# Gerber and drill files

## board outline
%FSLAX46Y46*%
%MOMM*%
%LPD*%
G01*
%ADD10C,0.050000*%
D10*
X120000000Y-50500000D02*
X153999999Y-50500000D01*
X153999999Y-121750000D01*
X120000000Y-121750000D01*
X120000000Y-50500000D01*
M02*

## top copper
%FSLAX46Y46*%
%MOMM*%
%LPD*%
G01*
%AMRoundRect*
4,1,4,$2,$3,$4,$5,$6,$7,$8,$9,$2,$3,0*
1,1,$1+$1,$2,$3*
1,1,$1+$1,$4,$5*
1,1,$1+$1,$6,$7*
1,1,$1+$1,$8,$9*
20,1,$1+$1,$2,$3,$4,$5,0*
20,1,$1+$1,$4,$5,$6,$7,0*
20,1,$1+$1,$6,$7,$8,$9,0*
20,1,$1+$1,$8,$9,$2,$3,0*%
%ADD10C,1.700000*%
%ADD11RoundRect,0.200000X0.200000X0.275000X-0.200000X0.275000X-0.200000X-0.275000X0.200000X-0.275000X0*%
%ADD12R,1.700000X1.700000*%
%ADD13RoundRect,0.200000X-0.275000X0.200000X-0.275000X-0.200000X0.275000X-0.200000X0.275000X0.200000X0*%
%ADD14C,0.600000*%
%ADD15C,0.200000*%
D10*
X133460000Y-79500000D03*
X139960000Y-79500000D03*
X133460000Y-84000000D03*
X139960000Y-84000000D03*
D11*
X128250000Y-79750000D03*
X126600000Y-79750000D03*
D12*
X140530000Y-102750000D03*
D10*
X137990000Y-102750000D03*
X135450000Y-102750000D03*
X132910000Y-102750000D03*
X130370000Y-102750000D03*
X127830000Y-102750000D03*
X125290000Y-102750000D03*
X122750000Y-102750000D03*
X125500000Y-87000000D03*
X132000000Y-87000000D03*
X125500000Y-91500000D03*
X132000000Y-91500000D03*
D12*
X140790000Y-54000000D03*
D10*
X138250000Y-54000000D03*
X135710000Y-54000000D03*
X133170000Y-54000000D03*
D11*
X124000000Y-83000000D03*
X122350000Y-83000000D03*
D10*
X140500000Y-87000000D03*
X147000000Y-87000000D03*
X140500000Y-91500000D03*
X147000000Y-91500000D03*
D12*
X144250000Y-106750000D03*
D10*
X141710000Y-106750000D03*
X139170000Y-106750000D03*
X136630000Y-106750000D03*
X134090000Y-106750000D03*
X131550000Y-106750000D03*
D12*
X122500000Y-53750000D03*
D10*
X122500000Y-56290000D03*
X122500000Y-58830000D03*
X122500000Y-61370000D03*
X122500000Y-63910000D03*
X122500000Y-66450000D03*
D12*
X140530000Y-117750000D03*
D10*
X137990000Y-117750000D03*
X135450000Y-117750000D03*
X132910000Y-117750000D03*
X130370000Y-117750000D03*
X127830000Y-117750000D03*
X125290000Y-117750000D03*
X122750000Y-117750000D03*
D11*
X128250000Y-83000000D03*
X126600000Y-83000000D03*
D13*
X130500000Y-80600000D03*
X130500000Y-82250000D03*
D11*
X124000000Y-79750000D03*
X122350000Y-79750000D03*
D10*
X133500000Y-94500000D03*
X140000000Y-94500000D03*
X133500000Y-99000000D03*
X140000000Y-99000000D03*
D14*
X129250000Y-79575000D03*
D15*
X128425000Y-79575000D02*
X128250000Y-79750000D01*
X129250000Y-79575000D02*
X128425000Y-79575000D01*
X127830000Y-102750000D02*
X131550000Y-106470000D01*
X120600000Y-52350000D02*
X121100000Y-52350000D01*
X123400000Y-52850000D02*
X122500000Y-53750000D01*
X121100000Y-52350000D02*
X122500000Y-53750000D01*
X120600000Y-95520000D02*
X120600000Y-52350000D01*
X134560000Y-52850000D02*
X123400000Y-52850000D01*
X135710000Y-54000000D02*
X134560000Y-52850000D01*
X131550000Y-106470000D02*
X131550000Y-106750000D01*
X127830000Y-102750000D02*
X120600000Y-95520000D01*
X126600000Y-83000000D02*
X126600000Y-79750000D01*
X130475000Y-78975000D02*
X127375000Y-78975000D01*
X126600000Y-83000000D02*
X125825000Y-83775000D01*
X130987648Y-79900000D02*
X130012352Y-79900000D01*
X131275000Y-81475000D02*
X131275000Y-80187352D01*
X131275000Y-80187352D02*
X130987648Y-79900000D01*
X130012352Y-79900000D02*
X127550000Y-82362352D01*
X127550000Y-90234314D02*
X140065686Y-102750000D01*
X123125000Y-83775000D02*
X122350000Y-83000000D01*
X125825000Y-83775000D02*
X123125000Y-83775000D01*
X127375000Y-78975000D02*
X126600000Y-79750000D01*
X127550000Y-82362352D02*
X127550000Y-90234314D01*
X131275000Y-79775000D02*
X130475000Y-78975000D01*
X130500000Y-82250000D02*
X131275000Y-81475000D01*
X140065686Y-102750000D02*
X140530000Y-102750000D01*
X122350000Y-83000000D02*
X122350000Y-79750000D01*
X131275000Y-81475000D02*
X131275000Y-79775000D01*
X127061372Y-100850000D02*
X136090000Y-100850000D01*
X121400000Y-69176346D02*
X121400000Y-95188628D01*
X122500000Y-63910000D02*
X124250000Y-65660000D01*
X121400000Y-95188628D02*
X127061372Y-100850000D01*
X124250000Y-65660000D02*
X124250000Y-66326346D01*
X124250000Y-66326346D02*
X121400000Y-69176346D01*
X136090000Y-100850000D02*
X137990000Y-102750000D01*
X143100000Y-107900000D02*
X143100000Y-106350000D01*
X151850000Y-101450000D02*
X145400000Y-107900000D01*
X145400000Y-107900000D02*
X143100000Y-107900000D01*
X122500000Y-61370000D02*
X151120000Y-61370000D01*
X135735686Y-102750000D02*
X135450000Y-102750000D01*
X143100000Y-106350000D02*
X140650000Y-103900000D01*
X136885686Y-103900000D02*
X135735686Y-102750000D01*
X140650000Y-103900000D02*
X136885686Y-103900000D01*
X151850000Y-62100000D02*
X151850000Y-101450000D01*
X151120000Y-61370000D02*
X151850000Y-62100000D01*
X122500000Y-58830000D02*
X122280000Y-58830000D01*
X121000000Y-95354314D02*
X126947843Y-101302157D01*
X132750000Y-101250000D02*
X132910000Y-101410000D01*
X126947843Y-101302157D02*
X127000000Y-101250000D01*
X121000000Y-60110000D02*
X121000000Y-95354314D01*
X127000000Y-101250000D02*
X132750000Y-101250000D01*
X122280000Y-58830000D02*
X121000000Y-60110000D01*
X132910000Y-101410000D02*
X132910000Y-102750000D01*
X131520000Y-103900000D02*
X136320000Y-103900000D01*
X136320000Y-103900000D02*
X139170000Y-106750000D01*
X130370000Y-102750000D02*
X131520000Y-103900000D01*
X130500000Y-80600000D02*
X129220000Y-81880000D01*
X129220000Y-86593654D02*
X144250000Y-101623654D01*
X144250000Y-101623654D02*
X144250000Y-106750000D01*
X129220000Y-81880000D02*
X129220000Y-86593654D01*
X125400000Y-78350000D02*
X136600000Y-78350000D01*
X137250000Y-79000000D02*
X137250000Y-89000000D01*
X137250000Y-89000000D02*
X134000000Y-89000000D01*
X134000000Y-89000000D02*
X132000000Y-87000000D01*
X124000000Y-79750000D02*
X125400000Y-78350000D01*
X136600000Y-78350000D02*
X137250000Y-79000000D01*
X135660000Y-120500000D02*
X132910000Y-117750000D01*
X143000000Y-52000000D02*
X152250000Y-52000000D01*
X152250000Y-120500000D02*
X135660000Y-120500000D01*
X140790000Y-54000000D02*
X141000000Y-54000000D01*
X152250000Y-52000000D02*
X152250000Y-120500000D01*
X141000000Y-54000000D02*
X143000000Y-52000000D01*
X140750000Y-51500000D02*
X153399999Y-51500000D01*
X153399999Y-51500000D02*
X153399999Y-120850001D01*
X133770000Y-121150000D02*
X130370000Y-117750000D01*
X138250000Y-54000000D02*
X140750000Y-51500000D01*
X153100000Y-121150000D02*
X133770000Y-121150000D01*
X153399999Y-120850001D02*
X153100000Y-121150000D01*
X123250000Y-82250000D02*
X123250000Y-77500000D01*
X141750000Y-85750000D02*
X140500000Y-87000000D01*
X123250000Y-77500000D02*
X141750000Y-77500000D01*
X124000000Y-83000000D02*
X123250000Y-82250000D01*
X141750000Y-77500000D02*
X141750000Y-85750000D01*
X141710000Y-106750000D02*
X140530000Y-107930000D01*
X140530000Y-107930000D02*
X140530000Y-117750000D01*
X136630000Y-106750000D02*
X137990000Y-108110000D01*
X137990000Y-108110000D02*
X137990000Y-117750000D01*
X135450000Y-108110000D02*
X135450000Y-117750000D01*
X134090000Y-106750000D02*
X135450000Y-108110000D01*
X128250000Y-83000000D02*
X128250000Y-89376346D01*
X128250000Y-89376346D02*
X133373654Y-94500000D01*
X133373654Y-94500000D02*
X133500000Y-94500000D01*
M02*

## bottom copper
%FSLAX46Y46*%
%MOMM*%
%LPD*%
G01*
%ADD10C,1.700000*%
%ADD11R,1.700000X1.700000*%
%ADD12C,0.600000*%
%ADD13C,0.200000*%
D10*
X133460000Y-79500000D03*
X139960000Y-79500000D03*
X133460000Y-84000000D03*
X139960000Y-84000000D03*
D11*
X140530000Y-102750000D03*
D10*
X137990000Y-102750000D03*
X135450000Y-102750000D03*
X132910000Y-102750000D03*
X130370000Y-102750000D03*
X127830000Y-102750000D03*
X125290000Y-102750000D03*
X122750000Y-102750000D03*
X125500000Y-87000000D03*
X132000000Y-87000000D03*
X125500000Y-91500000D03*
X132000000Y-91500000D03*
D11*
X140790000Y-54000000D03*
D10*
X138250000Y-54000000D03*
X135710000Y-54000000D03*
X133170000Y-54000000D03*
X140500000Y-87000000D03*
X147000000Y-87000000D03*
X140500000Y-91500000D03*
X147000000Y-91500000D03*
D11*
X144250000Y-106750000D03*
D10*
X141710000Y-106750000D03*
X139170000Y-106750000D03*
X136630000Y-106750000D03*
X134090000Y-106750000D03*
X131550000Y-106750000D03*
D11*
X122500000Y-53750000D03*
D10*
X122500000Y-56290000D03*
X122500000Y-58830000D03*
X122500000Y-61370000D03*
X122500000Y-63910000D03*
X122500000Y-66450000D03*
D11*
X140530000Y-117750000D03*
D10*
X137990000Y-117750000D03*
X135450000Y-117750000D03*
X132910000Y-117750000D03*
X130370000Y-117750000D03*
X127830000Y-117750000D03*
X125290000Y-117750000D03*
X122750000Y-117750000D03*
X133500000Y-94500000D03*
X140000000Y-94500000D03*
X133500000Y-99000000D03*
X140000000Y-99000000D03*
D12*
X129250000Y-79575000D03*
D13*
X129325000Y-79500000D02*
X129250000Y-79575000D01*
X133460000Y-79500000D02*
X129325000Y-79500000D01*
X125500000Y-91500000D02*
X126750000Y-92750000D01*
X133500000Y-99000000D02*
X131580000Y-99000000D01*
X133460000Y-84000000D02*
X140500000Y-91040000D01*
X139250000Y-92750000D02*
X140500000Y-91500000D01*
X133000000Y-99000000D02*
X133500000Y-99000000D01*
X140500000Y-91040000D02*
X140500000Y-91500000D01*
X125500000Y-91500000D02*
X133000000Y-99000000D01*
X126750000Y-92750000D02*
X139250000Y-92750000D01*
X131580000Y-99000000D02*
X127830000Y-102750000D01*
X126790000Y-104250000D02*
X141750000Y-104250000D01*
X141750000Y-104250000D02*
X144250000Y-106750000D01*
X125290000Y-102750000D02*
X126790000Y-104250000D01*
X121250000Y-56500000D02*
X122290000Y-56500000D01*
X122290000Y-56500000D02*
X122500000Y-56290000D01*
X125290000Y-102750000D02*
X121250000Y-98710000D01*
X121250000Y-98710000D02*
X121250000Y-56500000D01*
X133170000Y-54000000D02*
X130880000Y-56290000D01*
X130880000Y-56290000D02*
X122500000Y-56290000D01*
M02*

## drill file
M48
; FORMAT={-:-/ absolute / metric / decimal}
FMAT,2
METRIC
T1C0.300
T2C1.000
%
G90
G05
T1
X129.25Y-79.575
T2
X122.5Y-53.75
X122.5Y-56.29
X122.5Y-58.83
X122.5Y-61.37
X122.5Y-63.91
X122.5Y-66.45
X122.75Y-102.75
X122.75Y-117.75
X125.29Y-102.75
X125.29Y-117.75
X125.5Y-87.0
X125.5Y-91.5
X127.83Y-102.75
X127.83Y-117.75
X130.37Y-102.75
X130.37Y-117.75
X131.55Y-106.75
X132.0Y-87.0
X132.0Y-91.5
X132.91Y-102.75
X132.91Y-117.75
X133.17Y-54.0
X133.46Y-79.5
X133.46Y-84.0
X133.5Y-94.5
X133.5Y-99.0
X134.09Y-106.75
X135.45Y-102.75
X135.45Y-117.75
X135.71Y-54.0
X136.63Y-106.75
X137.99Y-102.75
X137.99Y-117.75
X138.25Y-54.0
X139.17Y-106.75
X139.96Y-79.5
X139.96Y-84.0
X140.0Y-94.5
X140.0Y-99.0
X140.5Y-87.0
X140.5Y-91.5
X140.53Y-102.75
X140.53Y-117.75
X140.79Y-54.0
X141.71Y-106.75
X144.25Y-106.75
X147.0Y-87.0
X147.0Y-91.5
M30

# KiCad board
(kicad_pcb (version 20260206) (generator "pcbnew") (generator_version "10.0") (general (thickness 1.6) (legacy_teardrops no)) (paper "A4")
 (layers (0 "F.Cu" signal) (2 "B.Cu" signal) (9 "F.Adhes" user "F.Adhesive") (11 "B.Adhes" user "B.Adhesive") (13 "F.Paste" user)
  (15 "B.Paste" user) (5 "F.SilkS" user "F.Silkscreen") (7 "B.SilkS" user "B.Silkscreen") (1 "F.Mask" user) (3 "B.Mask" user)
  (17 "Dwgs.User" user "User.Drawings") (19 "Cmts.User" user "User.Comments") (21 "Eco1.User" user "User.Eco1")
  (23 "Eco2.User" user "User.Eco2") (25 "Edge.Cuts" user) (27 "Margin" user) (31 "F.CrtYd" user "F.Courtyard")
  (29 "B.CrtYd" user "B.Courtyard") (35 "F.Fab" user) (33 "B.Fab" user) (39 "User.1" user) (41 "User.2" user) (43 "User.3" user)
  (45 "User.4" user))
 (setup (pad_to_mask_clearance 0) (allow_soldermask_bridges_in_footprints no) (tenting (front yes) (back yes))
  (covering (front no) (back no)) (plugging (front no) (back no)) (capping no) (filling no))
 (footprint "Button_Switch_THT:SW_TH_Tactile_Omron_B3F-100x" (layer "F.Cu") (at 133.46 79.5)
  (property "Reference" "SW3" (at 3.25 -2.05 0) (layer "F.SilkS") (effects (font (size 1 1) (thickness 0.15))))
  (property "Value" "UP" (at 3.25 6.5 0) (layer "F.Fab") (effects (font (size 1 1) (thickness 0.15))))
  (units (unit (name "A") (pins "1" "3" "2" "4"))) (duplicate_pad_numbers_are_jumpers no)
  (pad "1" thru_hole circle (at 0 0) (size 1.7 1.7) (drill 1) (layers "*.Cu" "*.Mask") (remove_unused_layers no) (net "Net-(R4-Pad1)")
   (thermal_bridge_angle 90))
  (pad "1" thru_hole circle (at 6.5 0) (size 1.7 1.7) (drill 1) (layers "*.Cu" "*.Mask") (remove_unused_layers no) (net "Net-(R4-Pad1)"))
  (pad "2" thru_hole circle (at 0 4.5) (size 1.7 1.7) (drill 1) (layers "*.Cu" "*.Mask") (remove_unused_layers no) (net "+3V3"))
  (pad "2" thru_hole circle (at 6.5 4.5) (size 1.7 1.7) (drill 1) (layers "*.Cu" "*.Mask") (remove_unused_layers no)
   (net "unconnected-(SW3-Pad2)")))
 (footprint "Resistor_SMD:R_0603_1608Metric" (layer "F.Cu") (at 127.425 79.75 180)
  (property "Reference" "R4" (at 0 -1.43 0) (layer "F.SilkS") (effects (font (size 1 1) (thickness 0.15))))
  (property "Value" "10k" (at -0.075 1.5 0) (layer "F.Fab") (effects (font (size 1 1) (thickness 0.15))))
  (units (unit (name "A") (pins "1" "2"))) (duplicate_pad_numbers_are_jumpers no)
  (pad "1" smd roundrect (at -0.825 0 180) (size 0.8 0.95) (layers "F.Cu" "F.Mask" "F.Paste") (roundrect_rratio 0.25) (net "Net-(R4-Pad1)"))
  (pad "2" smd roundrect (at 0.825 0 180) (size 0.8 0.95) (layers "F.Cu" "F.Mask" "F.Paste") (roundrect_rratio 0.25) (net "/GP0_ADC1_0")))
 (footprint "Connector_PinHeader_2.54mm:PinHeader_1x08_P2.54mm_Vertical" (layer "F.Cu") (at 140.53 102.75 -90)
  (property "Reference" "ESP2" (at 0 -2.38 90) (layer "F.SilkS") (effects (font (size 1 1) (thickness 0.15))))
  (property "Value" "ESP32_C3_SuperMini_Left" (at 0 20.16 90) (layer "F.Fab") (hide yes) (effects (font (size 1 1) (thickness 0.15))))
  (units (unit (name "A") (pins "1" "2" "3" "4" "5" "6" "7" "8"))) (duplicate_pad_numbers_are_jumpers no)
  (pad "1" thru_hole rect (at 0 0 270) (size 1.7 1.7) (drill 1) (layers "*.Cu" "*.Mask") (remove_unused_layers no) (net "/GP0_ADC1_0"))
  (pad "2" thru_hole circle (at 0 2.54 270) (size 1.7 1.7) (drill 1) (layers "*.Cu" "*.Mask") (remove_unused_layers no) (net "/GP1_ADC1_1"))
  (pad "3" thru_hole circle (at 0 5.08 270) (size 1.7 1.7) (drill 1) (layers "*.Cu" "*.Mask") (remove_unused_layers no) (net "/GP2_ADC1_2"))
  (pad "4" thru_hole circle (at 0 7.62 270) (size 1.7 1.7) (drill 1) (layers "*.Cu" "*.Mask") (remove_unused_layers no) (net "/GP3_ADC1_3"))
  (pad "5" thru_hole circle (at 0 10.16 270) (size 1.7 1.7) (drill 1) (layers "*.Cu" "*.Mask") (remove_unused_layers no) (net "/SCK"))
  (pad "6" thru_hole circle (at 0 12.7 270) (size 1.7 1.7) (drill 1) (layers "*.Cu" "*.Mask") (remove_unused_layers no) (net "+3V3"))
  (pad "7" thru_hole circle (at 0 15.24 270) (size 1.7 1.7) (drill 1) (layers "*.Cu" "*.Mask") (remove_unused_layers no) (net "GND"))
  (pad "8" thru_hole circle (at 0 17.78 270) (size 1.7 1.7) (drill 1) (layers "*.Cu" "*.Mask") (remove_unused_layers no)
   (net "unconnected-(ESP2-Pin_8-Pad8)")))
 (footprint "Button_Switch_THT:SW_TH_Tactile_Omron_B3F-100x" (layer "F.Cu") (at 125.5 87)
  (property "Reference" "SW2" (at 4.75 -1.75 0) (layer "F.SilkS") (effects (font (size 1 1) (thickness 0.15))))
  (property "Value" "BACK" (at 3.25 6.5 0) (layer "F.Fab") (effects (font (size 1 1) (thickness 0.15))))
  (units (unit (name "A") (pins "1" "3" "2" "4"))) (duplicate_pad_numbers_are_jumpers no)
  (pad "1" thru_hole circle (at 0 0) (size 1.7 1.7) (drill 1) (layers "*.Cu" "*.Mask") (remove_unused_layers no) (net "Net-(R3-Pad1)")
   (thermal_bridge_angle 90))
  (pad "1" thru_hole circle (at 6.5 0) (size 1.7 1.7) (drill 1) (layers "*.Cu" "*.Mask") (remove_unused_layers no) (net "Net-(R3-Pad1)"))
  (pad "2" thru_hole circle (at 0 4.5) (size 1.7 1.7) (drill 1) (layers "*.Cu" "*.Mask") (remove_unused_layers no) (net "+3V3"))
  (pad "2" thru_hole circle (at 6.5 4.5) (size 1.7 1.7) (drill 1) (layers "*.Cu" "*.Mask") (remove_unused_layers no)
   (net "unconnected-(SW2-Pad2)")))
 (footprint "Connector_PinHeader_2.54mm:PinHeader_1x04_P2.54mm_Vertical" (layer "F.Cu") (at 140.79 54 -90)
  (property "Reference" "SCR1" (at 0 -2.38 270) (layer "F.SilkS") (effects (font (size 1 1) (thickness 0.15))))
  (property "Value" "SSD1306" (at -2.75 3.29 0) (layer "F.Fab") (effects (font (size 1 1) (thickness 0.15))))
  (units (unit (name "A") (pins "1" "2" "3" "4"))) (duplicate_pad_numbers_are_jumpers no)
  (pad "1" thru_hole rect (at 0 0 270) (size 1.7 1.7) (drill 1) (layers "*.Cu" "*.Mask") (remove_unused_layers no) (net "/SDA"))
  (pad "2" thru_hole circle (at 0 2.54 270) (size 1.7 1.7) (drill 1) (layers "*.Cu" "*.Mask") (remove_unused_layers no) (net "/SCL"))
  (pad "3" thru_hole circle (at 0 5.08 270) (size 1.7 1.7) (drill 1) (layers "*.Cu" "*.Mask") (remove_unused_layers no) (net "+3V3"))
  (pad "4" thru_hole circle (at 0 7.62 270) (size 1.7 1.7) (drill 1) (layers "*.Cu" "*.Mask") (remove_unused_layers no) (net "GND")))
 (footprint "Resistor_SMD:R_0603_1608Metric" (layer "F.Cu") (at 123.175 83 180)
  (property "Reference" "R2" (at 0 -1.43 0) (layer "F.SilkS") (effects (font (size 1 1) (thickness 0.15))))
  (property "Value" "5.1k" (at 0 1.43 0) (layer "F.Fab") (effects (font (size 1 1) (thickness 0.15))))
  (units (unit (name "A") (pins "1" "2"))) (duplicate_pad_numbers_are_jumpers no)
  (pad "1" smd roundrect (at -0.825 0 180) (size 0.8 0.95) (layers "F.Cu" "F.Mask" "F.Paste") (roundrect_rratio 0.25) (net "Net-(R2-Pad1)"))
  (pad "2" smd roundrect (at 0.825 0 180) (size 0.8 0.95) (layers "F.Cu" "F.Mask" "F.Paste") (roundrect_rratio 0.25) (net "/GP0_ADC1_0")))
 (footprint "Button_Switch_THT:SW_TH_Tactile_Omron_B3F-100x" (layer "F.Cu") (at 140.5 87)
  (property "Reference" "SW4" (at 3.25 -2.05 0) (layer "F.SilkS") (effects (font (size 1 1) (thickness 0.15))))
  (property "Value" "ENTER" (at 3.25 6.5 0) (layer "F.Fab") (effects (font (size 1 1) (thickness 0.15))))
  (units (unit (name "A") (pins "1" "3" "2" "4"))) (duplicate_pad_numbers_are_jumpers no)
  (pad "1" thru_hole circle (at 0 0) (size 1.7 1.7) (drill 1) (layers "*.Cu" "*.Mask") (remove_unused_layers no) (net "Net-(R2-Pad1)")
   (thermal_bridge_angle 90))
  (pad "1" thru_hole circle (at 6.5 0) (size 1.7 1.7) (drill 1) (layers "*.Cu" "*.Mask") (remove_unused_layers no) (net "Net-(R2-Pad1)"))
  (pad "2" thru_hole circle (at 0 4.5) (size 1.7 1.7) (drill 1) (layers "*.Cu" "*.Mask") (remove_unused_layers no) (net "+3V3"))
  (pad "2" thru_hole circle (at 6.5 4.5) (size 1.7 1.7) (drill 1) (layers "*.Cu" "*.Mask") (remove_unused_layers no)
   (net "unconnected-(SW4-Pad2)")))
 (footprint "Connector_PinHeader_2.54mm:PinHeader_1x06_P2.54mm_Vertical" (layer "F.Cu") (at 144.25 106.75 -90)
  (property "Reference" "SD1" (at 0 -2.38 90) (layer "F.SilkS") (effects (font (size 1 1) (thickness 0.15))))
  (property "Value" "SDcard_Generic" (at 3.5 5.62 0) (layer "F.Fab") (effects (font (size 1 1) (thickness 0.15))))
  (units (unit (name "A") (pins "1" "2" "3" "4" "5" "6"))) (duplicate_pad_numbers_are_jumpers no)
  (pad "1" thru_hole rect (at 0 0 270) (size 1.7 1.7) (drill 1) (layers "*.Cu" "*.Mask") (remove_unused_layers no) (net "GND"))
  (pad "2" thru_hole circle (at 0 2.54 270) (size 1.7 1.7) (drill 1) (layers "*.Cu" "*.Mask") (remove_unused_layers no) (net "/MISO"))
  (pad "3" thru_hole circle (at 0 5.08 270) (size 1.7 1.7) (drill 1) (layers "*.Cu" "*.Mask") (remove_unused_layers no) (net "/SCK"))
  (pad "4" thru_hole circle (at 0 7.62 270) (size 1.7 1.7) (drill 1) (layers "*.Cu" "*.Mask") (remove_unused_layers no) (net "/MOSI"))
  (pad "5" thru_hole circle (at 0 10.16 270) (size 1.7 1.7) (drill 1) (layers "*.Cu" "*.Mask") (remove_unused_layers no) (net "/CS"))
  (pad "6" thru_hole circle (at 0 12.7 270) (size 1.7 1.7) (drill 1) (layers "*.Cu" "*.Mask") (remove_unused_layers no) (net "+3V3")))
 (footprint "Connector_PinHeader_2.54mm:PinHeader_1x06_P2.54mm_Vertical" (layer "F.Cu") (at 122.5 53.75)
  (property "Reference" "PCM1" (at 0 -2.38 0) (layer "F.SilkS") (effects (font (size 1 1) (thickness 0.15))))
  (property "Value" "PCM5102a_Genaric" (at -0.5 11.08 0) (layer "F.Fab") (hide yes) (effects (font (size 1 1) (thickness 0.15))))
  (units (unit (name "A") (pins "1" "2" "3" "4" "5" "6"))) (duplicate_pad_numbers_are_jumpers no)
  (pad "1" thru_hole rect (at 0 0) (size 1.7 1.7) (drill 1) (layers "*.Cu" "*.Mask") (remove_unused_layers no) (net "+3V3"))
  (pad "2" thru_hole circle (at 0 2.54) (size 1.7 1.7) (drill 1) (layers "*.Cu" "*.Mask") (remove_unused_layers no) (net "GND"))
  (pad "3" thru_hole circle (at 0 5.08) (size 1.7 1.7) (drill 1) (layers "*.Cu" "*.Mask") (remove_unused_layers no) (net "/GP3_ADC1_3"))
  (pad "4" thru_hole circle (at 0 7.62) (size 1.7 1.7) (drill 1) (layers "*.Cu" "*.Mask") (remove_unused_layers no) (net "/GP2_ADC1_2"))
  (pad "5" thru_hole circle (at 0 10.16) (size 1.7 1.7) (drill 1) (layers "*.Cu" "*.Mask") (remove_unused_layers no) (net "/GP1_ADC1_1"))
  (pad "6" thru_hole circle (at 0 12.7) (size 1.7 1.7) (drill 1) (layers "*.Cu" "*.Mask") (remove_unused_layers no)
   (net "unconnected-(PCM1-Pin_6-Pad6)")))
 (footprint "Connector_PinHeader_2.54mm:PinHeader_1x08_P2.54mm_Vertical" (layer "F.Cu") (at 140.53 117.75 -90)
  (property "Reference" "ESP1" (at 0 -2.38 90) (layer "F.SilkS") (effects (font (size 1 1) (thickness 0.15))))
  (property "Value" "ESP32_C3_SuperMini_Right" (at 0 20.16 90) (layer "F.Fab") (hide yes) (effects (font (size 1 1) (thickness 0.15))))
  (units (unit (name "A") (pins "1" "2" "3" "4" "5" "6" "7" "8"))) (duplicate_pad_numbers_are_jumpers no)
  (pad "1" thru_hole rect (at 0 0 270) (size 1.7 1.7) (drill 1) (layers "*.Cu" "*.Mask") (remove_unused_layers no) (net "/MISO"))
  (pad "2" thru_hole circle (at 0 2.54 270) (size 1.7 1.7) (drill 1) (layers "*.Cu" "*.Mask") (remove_unused_layers no) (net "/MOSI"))
  (pad "3" thru_hole circle (at 0 5.08 270) (size 1.7 1.7) (drill 1) (layers "*.Cu" "*.Mask") (remove_unused_layers no) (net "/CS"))
  (pad "4" thru_hole circle (at 0 7.62 270) (size 1.7 1.7) (drill 1) (layers "*.Cu" "*.Mask") (remove_unused_layers no) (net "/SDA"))
  (pad "5" thru_hole circle (at 0 10.16 270) (size 1.7 1.7) (drill 1) (layers "*.Cu" "*.Mask") (remove_unused_layers no) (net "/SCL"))
  (pad "6" thru_hole circle (at 0 12.7 270) (size 1.7 1.7) (drill 1) (layers "*.Cu" "*.Mask") (remove_unused_layers no)
   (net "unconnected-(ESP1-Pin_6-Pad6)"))
  (pad "7" thru_hole circle (at 0 15.24 270) (size 1.7 1.7) (drill 1) (layers "*.Cu" "*.Mask") (remove_unused_layers no)
   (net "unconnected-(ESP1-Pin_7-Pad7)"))
  (pad "8" thru_hole circle (at 0 17.78 270) (size 1.7 1.7) (drill 1) (layers "*.Cu" "*.Mask") (remove_unused_layers no)
   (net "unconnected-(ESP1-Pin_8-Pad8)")))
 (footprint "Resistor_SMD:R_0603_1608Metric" (layer "F.Cu") (at 127.425 83 180)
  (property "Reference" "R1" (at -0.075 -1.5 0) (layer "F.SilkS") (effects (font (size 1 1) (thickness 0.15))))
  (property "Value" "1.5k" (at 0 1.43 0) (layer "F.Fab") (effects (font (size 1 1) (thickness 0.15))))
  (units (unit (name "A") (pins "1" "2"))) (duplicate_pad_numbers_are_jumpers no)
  (pad "1" smd roundrect (at -0.825 0 180) (size 0.8 0.95) (layers "F.Cu" "F.Mask" "F.Paste") (roundrect_rratio 0.25) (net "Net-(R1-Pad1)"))
  (pad "2" smd roundrect (at 0.825 0 180) (size 0.8 0.95) (layers "F.Cu" "F.Mask" "F.Paste") (roundrect_rratio 0.25) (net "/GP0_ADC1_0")))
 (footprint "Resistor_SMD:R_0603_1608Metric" (layer "F.Cu") (at 130.5 81.425 -90)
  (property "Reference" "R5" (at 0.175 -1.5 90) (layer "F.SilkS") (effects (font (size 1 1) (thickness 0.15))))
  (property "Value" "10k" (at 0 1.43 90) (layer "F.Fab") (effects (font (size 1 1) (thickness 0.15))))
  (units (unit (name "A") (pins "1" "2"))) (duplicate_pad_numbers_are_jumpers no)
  (pad "1" smd roundrect (at -0.825 0 270) (size 0.8 0.95) (layers "F.Cu" "F.Mask" "F.Paste") (roundrect_rratio 0.25) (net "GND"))
  (pad "2" smd roundrect (at 0.825 0 270) (size 0.8 0.95) (layers "F.Cu" "F.Mask" "F.Paste") (roundrect_rratio 0.25) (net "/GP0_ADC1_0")))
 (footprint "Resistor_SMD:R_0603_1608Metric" (layer "F.Cu") (at 123.175 79.75 180)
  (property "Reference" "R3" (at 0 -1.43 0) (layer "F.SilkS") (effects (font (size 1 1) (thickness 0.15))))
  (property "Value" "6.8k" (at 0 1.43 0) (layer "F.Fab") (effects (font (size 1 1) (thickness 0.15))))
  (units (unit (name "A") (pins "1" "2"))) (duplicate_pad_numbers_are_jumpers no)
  (pad "1" smd roundrect (at -0.825 0 180) (size 0.8 0.95) (layers "F.Cu" "F.Mask" "F.Paste") (roundrect_rratio 0.25) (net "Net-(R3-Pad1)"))
  (pad "2" smd roundrect (at 0.825 0 180) (size 0.8 0.95) (layers "F.Cu" "F.Mask" "F.Paste") (roundrect_rratio 0.25) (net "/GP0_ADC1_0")))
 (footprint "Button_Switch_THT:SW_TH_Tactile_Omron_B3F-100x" (layer "F.Cu") (at 133.5 94.5)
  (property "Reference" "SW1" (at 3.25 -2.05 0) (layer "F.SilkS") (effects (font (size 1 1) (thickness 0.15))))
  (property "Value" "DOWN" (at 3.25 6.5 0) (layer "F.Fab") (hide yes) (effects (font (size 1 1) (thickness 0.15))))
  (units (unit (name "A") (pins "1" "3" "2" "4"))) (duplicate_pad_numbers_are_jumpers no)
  (pad "1" thru_hole circle (at 0 0) (size 1.7 1.7) (drill 1) (layers "*.Cu" "*.Mask") (remove_unused_layers no) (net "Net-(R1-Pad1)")
   (thermal_bridge_angle 90))
  (pad "1" thru_hole circle (at 6.5 0) (size 1.7 1.7) (drill 1) (layers "*.Cu" "*.Mask") (remove_unused_layers no) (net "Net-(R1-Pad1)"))
  (pad "2" thru_hole circle (at 0 4.5) (size 1.7 1.7) (drill 1) (layers "*.Cu" "*.Mask") (remove_unused_layers no) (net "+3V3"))
  (pad "2" thru_hole circle (at 6.5 4.5) (size 1.7 1.7) (drill 1) (layers "*.Cu" "*.Mask") (remove_unused_layers no)
   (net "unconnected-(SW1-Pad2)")))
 (gr_rect (start 120 50.5) (end 153.999999 121.75) (stroke (width 0.05) (type default)) (fill no) (layer "Edge.Cuts"))
 (segment (start 128.425 79.575) (end 128.25 79.75) (width 0.2) (layer "F.Cu") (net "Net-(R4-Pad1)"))
 (segment (start 129.25 79.575) (end 128.425 79.575) (width 0.2) (layer "F.Cu") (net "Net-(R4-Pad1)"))
 (via (at 129.25 79.575) (size 0.6) (drill 0.3) (layers "F.Cu" "B.Cu") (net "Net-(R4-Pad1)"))
 (segment (start 129.325 79.5) (end 129.25 79.575) (width 0.2) (layer "B.Cu") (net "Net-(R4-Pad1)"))
 (segment (start 133.46 79.5) (end 129.325 79.5) (width 0.2) (layer "B.Cu") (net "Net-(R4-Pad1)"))
 (segment (start 127.83 102.75) (end 131.55 106.47) (width 0.2) (layer "F.Cu") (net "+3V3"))
 (segment (start 120.6 52.35) (end 121.1 52.35) (width 0.2) (layer "F.Cu") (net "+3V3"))
 (segment (start 123.4 52.85) (end 122.5 53.75) (width 0.2) (layer "F.Cu") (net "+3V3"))
 (segment (start 121.1 52.35) (end 122.5 53.75) (width 0.2) (layer "F.Cu") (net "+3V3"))
 (segment (start 120.6 95.52) (end 120.6 52.35) (width 0.2) (layer "F.Cu") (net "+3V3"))
 (segment (start 134.56 52.85) (end 123.4 52.85) (width 0.2) (layer "F.Cu") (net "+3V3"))
 (segment (start 135.71 54) (end 134.56 52.85) (width 0.2) (layer "F.Cu") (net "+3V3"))
 (segment (start 131.55 106.47) (end 131.55 106.75) (width 0.2) (layer "F.Cu") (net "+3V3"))
 (segment (start 127.83 102.75) (end 120.6 95.52) (width 0.2) (layer "F.Cu") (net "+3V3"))
 (segment (start 125.5 91.5) (end 126.75 92.75) (width 0.2) (layer "B.Cu") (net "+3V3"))
 (segment (start 133.5 99) (end 131.58 99) (width 0.2) (layer "B.Cu") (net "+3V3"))
 (segment (start 133.46 84) (end 140.5 91.04) (width 0.2) (layer "B.Cu") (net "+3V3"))
 (segment (start 139.25 92.75) (end 140.5 91.5) (width 0.2) (layer "B.Cu") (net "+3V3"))
 (segment (start 133 99) (end 133.5 99) (width 0.2) (layer "B.Cu") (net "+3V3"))
 (segment (start 140.5 91.04) (end 140.5 91.5) (width 0.2) (layer "B.Cu") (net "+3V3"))
 (segment (start 125.5 91.5) (end 133 99) (width 0.2) (layer "B.Cu") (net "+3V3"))
 (segment (start 126.75 92.75) (end 139.25 92.75) (width 0.2) (layer "B.Cu") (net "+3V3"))
 (segment (start 131.58 99) (end 127.83 102.75) (width 0.2) (layer "B.Cu") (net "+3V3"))
 (segment (start 126.6 83) (end 126.6 79.75) (width 0.2) (layer "F.Cu") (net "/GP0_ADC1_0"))
 (segment (start 130.475 78.975) (end 127.375 78.975) (width 0.2) (layer "F.Cu") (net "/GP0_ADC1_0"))
 (segment (start 126.6 83) (end 125.825 83.775) (width 0.2) (layer "F.Cu") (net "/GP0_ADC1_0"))
 (segment (start 130.987648 79.9) (end 130.012352 79.9) (width 0.2) (layer "F.Cu") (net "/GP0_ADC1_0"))
 (segment (start 131.275 81.475) (end 131.275 80.187352) (width 0.2) (layer "F.Cu") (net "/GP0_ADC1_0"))
 (segment (start 131.275 80.187352) (end 130.987648 79.9) (width 0.2) (layer "F.Cu") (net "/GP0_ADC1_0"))
 (segment (start 130.012352 79.9) (end 127.55 82.362352) (width 0.2) (layer "F.Cu") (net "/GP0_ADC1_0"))
 (segment (start 127.55 90.234314) (end 140.065686 102.75) (width 0.2) (layer "F.Cu") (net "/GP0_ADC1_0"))
 (segment (start 123.125 83.775) (end 122.35 83) (width 0.2) (layer "F.Cu") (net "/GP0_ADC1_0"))
 (segment (start 125.825 83.775) (end 123.125 83.775) (width 0.2) (layer "F.Cu") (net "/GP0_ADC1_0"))
 (segment (start 127.375 78.975) (end 126.6 79.75) (width 0.2) (layer "F.Cu") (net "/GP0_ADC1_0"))
 (segment (start 127.55 82.362352) (end 127.55 90.234314) (width 0.2) (layer "F.Cu") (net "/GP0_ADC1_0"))
 (segment (start 131.275 79.775) (end 130.475 78.975) (width 0.2) (layer "F.Cu") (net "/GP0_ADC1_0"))
 (segment (start 130.5 82.25) (end 131.275 81.475) (width 0.2) (layer "F.Cu") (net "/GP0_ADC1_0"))
 (segment (start 140.065686 102.75) (end 140.53 102.75) (width 0.2) (layer "F.Cu") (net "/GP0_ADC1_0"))
 (segment (start 122.35 83) (end 122.35 79.75) (width 0.2) (layer "F.Cu") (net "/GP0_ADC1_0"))
 (segment (start 131.275 81.475) (end 131.275 79.775) (width 0.2) (layer "F.Cu") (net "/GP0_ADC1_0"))
 (segment (start 127.061372 100.85) (end 136.09 100.85) (width 0.2) (layer "F.Cu") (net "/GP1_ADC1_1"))
 (segment (start 121.4 69.176346) (end 121.4 95.188628) (width 0.2) (layer "F.Cu") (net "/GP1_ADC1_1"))
 (segment (start 122.5 63.91) (end 124.25 65.66) (width 0.2) (layer "F.Cu") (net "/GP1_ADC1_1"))
 (segment (start 121.4 95.188628) (end 127.061372 100.85) (width 0.2) (layer "F.Cu") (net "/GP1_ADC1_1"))
 (segment (start 124.25 65.66) (end 124.25 66.326346) (width 0.2) (layer "F.Cu") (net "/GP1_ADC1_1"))
 (segment (start 124.25 66.326346) (end 121.4 69.176346) (width 0.2) (layer "F.Cu") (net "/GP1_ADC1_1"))
 (segment (start 136.09 100.85) (end 137.99 102.75) (width 0.2) (layer "F.Cu") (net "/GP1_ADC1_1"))
 (segment (start 143.1 107.9) (end 143.1 106.35) (width 0.2) (layer "F.Cu") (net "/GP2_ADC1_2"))
 (segment (start 151.85 101.45) (end 145.4 107.9) (width 0.2) (layer "F.Cu") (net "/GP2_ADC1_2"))
 (segment (start 145.4 107.9) (end 143.1 107.9) (width 0.2) (layer "F.Cu") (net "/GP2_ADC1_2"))
 (segment (start 122.5 61.37) (end 151.12 61.37) (width 0.2) (layer "F.Cu") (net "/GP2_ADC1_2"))
 (segment (start 135.735686 102.75) (end 135.45 102.75) (width 0.2) (layer "F.Cu") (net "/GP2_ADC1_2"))
 (segment (start 143.1 106.35) (end 140.65 103.9) (width 0.2) (layer "F.Cu") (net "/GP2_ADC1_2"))
 (segment (start 136.885686 103.9) (end 135.735686 102.75) (width 0.2) (layer "F.Cu") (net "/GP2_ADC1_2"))
 (segment (start 140.65 103.9) (end 136.885686 103.9) (width 0.2) (layer "F.Cu") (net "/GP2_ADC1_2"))
 (segment (start 151.85 62.1) (end 151.85 101.45) (width 0.2) (layer "F.Cu") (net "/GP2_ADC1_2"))
 (segment (start 151.12 61.37) (end 151.85 62.1) (width 0.2) (layer "F.Cu") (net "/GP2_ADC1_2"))
 (segment (start 122.5 58.83) (end 122.28 58.83) (width 0.2) (layer "F.Cu") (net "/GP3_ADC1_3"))
 (segment (start 121 95.354314) (end 126.947843 101.302157) (width 0.2) (layer "F.Cu") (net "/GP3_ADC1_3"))
 (segment (start 132.75 101.25) (end 132.91 101.41) (width 0.2) (layer "F.Cu") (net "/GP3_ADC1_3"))
 (segment (start 126.947843 101.302157) (end 127 101.25) (width 0.2) (layer "F.Cu") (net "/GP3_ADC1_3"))
 (segment (start 121 60.11) (end 121 95.354314) (width 0.2) (layer "F.Cu") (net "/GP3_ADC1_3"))
 (segment (start 127 101.25) (end 132.75 101.25) (width 0.2) (layer "F.Cu") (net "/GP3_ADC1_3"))
 (segment (start 122.28 58.83) (end 121 60.11) (width 0.2) (layer "F.Cu") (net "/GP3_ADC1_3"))
 (segment (start 132.91 101.41) (end 132.91 102.75) (width 0.2) (layer "F.Cu") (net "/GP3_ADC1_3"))
 (segment (start 131.52 103.9) (end 136.32 103.9) (width 0.2) (layer "F.Cu") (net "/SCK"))
 (segment (start 136.32 103.9) (end 139.17 106.75) (width 0.2) (layer "F.Cu") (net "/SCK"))
 (segment (start 130.37 102.75) (end 131.52 103.9) (width 0.2) (layer "F.Cu") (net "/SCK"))
 (segment (start 130.5 80.6) (end 129.22 81.88) (width 0.2) (layer "F.Cu") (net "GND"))
 (segment (start 129.22 86.593654) (end 144.25 101.623654) (width 0.2) (layer "F.Cu") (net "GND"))
 (segment (start 144.25 101.623654) (end 144.25 106.75) (width 0.2) (layer "F.Cu") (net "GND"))
 (segment (start 129.22 81.88) (end 129.22 86.593654) (width 0.2) (layer "F.Cu") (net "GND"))
 (segment (start 126.79 104.25) (end 141.75 104.25) (width 0.2) (layer "B.Cu") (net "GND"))
 (segment (start 141.75 104.25) (end 144.25 106.75) (width 0.2) (layer "B.Cu") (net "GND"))
 (segment (start 125.29 102.75) (end 126.79 104.25) (width 0.2) (layer "B.Cu") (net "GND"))
 (segment (start 121.25 56.5) (end 122.29 56.5) (width 0.2) (layer "B.Cu") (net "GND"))
 (segment (start 122.29 56.5) (end 122.5 56.29) (width 0.2) (layer "B.Cu") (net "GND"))
 (segment (start 125.29 102.75) (end 121.25 98.71) (width 0.2) (layer "B.Cu") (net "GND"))
 (segment (start 121.25 98.71) (end 121.25 56.5) (width 0.2) (layer "B.Cu") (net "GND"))
 (segment (start 133.17 54) (end 130.88 56.29) (width 0.2) (layer "B.Cu") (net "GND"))
 (segment (start 130.88 56.29) (end 122.5 56.29) (width 0.2) (layer "B.Cu") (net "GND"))
 (segment (start 125.4 78.35) (end 136.6 78.35) (width 0.2) (layer "F.Cu") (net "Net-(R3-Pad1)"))
 (segment (start 137.25 79) (end 137.25 89) (width 0.2) (layer "F.Cu") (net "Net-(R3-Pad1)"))
 (segment (start 137.25 89) (end 134 89) (width 0.2) (layer "F.Cu") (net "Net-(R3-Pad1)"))
 (segment (start 134 89) (end 132 87) (width 0.2) (layer "F.Cu") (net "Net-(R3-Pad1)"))
 (segment (start 124 79.75) (end 125.4 78.35) (width 0.2) (layer "F.Cu") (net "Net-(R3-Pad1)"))
 (segment (start 136.6 78.35) (end 137.25 79) (width 0.2) (layer "F.Cu") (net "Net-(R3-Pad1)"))
 (segment (start 135.66 120.5) (end 132.91 117.75) (width 0.2) (layer "F.Cu") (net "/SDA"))
 (segment (start 143 52) (end 152.25 52) (width 0.2) (layer "F.Cu") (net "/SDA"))
 (segment (start 152.25 120.5) (end 135.66 120.5) (width 0.2) (layer "F.Cu") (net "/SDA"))
 (segment (start 140.79 54) (end 141 54) (width 0.2) (layer "F.Cu") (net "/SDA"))
 (segment (start 152.25 52) (end 152.25 120.5) (width 0.2) (layer "F.Cu") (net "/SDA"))
 (segment (start 141 54) (end 143 52) (width 0.2) (layer "F.Cu") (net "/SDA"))
 (segment (start 140.75 51.5) (end 153.399999 51.5) (width 0.2) (layer "F.Cu") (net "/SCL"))
 (segment (start 153.399999 51.5) (end 153.399999 120.850001) (width 0.2) (layer "F.Cu") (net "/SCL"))
 (segment (start 133.77 121.15) (end 130.37 117.75) (width 0.2) (layer "F.Cu") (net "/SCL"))
 (segment (start 138.25 54) (end 140.75 51.5) (width 0.2) (layer "F.Cu") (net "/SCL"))
 (segment (start 153.1 121.15) (end 133.77 121.15) (width 0.2) (layer "F.Cu") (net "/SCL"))
 (segment (start 153.399999 120.850001) (end 153.1 121.15) (width 0.2) (layer "F.Cu") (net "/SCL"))
 (segment (start 123.25 82.25) (end 123.25 77.5) (width 0.2) (layer "F.Cu") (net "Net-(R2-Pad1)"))
 (segment (start 141.75 85.75) (end 140.5 87) (width 0.2) (layer "F.Cu") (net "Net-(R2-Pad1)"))
 (segment (start 123.25 77.5) (end 141.75 77.5) (width 0.2) (layer "F.Cu") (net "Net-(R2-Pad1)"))
 (segment (start 124 83) (end 123.25 82.25) (width 0.2) (layer "F.Cu") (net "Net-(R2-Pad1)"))
 (segment (start 141.75 77.5) (end 141.75 85.75) (width 0.2) (layer "F.Cu") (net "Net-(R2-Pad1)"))
 (segment (start 141.71 106.75) (end 140.53 107.93) (width 0.2) (layer "F.Cu") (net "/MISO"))
 (segment (start 140.53 107.93) (end 140.53 117.75) (width 0.2) (layer "F.Cu") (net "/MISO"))
 (segment (start 136.63 106.75) (end 137.99 108.11) (width 0.2) (layer "F.Cu") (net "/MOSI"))
 (segment (start 137.99 108.11) (end 137.99 117.75) (width 0.2) (layer "F.Cu") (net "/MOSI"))
 (segment (start 135.45 108.11) (end 135.45 117.75) (width 0.2) (layer "F.Cu") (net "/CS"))
 (segment (start 134.09 106.75) (end 135.45 108.11) (width 0.2) (layer "F.Cu") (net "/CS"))
 (segment (start 128.25 83) (end 128.25 89.376346) (width 0.2) (layer "F.Cu") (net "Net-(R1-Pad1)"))
 (segment (start 128.25 89.376346) (end 133.373654 94.5) (width 0.2) (layer "F.Cu") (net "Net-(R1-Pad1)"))
 (segment (start 133.373654 94.5) (end 133.5 94.5) (width 0.2) (layer "F.Cu") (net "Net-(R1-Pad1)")))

